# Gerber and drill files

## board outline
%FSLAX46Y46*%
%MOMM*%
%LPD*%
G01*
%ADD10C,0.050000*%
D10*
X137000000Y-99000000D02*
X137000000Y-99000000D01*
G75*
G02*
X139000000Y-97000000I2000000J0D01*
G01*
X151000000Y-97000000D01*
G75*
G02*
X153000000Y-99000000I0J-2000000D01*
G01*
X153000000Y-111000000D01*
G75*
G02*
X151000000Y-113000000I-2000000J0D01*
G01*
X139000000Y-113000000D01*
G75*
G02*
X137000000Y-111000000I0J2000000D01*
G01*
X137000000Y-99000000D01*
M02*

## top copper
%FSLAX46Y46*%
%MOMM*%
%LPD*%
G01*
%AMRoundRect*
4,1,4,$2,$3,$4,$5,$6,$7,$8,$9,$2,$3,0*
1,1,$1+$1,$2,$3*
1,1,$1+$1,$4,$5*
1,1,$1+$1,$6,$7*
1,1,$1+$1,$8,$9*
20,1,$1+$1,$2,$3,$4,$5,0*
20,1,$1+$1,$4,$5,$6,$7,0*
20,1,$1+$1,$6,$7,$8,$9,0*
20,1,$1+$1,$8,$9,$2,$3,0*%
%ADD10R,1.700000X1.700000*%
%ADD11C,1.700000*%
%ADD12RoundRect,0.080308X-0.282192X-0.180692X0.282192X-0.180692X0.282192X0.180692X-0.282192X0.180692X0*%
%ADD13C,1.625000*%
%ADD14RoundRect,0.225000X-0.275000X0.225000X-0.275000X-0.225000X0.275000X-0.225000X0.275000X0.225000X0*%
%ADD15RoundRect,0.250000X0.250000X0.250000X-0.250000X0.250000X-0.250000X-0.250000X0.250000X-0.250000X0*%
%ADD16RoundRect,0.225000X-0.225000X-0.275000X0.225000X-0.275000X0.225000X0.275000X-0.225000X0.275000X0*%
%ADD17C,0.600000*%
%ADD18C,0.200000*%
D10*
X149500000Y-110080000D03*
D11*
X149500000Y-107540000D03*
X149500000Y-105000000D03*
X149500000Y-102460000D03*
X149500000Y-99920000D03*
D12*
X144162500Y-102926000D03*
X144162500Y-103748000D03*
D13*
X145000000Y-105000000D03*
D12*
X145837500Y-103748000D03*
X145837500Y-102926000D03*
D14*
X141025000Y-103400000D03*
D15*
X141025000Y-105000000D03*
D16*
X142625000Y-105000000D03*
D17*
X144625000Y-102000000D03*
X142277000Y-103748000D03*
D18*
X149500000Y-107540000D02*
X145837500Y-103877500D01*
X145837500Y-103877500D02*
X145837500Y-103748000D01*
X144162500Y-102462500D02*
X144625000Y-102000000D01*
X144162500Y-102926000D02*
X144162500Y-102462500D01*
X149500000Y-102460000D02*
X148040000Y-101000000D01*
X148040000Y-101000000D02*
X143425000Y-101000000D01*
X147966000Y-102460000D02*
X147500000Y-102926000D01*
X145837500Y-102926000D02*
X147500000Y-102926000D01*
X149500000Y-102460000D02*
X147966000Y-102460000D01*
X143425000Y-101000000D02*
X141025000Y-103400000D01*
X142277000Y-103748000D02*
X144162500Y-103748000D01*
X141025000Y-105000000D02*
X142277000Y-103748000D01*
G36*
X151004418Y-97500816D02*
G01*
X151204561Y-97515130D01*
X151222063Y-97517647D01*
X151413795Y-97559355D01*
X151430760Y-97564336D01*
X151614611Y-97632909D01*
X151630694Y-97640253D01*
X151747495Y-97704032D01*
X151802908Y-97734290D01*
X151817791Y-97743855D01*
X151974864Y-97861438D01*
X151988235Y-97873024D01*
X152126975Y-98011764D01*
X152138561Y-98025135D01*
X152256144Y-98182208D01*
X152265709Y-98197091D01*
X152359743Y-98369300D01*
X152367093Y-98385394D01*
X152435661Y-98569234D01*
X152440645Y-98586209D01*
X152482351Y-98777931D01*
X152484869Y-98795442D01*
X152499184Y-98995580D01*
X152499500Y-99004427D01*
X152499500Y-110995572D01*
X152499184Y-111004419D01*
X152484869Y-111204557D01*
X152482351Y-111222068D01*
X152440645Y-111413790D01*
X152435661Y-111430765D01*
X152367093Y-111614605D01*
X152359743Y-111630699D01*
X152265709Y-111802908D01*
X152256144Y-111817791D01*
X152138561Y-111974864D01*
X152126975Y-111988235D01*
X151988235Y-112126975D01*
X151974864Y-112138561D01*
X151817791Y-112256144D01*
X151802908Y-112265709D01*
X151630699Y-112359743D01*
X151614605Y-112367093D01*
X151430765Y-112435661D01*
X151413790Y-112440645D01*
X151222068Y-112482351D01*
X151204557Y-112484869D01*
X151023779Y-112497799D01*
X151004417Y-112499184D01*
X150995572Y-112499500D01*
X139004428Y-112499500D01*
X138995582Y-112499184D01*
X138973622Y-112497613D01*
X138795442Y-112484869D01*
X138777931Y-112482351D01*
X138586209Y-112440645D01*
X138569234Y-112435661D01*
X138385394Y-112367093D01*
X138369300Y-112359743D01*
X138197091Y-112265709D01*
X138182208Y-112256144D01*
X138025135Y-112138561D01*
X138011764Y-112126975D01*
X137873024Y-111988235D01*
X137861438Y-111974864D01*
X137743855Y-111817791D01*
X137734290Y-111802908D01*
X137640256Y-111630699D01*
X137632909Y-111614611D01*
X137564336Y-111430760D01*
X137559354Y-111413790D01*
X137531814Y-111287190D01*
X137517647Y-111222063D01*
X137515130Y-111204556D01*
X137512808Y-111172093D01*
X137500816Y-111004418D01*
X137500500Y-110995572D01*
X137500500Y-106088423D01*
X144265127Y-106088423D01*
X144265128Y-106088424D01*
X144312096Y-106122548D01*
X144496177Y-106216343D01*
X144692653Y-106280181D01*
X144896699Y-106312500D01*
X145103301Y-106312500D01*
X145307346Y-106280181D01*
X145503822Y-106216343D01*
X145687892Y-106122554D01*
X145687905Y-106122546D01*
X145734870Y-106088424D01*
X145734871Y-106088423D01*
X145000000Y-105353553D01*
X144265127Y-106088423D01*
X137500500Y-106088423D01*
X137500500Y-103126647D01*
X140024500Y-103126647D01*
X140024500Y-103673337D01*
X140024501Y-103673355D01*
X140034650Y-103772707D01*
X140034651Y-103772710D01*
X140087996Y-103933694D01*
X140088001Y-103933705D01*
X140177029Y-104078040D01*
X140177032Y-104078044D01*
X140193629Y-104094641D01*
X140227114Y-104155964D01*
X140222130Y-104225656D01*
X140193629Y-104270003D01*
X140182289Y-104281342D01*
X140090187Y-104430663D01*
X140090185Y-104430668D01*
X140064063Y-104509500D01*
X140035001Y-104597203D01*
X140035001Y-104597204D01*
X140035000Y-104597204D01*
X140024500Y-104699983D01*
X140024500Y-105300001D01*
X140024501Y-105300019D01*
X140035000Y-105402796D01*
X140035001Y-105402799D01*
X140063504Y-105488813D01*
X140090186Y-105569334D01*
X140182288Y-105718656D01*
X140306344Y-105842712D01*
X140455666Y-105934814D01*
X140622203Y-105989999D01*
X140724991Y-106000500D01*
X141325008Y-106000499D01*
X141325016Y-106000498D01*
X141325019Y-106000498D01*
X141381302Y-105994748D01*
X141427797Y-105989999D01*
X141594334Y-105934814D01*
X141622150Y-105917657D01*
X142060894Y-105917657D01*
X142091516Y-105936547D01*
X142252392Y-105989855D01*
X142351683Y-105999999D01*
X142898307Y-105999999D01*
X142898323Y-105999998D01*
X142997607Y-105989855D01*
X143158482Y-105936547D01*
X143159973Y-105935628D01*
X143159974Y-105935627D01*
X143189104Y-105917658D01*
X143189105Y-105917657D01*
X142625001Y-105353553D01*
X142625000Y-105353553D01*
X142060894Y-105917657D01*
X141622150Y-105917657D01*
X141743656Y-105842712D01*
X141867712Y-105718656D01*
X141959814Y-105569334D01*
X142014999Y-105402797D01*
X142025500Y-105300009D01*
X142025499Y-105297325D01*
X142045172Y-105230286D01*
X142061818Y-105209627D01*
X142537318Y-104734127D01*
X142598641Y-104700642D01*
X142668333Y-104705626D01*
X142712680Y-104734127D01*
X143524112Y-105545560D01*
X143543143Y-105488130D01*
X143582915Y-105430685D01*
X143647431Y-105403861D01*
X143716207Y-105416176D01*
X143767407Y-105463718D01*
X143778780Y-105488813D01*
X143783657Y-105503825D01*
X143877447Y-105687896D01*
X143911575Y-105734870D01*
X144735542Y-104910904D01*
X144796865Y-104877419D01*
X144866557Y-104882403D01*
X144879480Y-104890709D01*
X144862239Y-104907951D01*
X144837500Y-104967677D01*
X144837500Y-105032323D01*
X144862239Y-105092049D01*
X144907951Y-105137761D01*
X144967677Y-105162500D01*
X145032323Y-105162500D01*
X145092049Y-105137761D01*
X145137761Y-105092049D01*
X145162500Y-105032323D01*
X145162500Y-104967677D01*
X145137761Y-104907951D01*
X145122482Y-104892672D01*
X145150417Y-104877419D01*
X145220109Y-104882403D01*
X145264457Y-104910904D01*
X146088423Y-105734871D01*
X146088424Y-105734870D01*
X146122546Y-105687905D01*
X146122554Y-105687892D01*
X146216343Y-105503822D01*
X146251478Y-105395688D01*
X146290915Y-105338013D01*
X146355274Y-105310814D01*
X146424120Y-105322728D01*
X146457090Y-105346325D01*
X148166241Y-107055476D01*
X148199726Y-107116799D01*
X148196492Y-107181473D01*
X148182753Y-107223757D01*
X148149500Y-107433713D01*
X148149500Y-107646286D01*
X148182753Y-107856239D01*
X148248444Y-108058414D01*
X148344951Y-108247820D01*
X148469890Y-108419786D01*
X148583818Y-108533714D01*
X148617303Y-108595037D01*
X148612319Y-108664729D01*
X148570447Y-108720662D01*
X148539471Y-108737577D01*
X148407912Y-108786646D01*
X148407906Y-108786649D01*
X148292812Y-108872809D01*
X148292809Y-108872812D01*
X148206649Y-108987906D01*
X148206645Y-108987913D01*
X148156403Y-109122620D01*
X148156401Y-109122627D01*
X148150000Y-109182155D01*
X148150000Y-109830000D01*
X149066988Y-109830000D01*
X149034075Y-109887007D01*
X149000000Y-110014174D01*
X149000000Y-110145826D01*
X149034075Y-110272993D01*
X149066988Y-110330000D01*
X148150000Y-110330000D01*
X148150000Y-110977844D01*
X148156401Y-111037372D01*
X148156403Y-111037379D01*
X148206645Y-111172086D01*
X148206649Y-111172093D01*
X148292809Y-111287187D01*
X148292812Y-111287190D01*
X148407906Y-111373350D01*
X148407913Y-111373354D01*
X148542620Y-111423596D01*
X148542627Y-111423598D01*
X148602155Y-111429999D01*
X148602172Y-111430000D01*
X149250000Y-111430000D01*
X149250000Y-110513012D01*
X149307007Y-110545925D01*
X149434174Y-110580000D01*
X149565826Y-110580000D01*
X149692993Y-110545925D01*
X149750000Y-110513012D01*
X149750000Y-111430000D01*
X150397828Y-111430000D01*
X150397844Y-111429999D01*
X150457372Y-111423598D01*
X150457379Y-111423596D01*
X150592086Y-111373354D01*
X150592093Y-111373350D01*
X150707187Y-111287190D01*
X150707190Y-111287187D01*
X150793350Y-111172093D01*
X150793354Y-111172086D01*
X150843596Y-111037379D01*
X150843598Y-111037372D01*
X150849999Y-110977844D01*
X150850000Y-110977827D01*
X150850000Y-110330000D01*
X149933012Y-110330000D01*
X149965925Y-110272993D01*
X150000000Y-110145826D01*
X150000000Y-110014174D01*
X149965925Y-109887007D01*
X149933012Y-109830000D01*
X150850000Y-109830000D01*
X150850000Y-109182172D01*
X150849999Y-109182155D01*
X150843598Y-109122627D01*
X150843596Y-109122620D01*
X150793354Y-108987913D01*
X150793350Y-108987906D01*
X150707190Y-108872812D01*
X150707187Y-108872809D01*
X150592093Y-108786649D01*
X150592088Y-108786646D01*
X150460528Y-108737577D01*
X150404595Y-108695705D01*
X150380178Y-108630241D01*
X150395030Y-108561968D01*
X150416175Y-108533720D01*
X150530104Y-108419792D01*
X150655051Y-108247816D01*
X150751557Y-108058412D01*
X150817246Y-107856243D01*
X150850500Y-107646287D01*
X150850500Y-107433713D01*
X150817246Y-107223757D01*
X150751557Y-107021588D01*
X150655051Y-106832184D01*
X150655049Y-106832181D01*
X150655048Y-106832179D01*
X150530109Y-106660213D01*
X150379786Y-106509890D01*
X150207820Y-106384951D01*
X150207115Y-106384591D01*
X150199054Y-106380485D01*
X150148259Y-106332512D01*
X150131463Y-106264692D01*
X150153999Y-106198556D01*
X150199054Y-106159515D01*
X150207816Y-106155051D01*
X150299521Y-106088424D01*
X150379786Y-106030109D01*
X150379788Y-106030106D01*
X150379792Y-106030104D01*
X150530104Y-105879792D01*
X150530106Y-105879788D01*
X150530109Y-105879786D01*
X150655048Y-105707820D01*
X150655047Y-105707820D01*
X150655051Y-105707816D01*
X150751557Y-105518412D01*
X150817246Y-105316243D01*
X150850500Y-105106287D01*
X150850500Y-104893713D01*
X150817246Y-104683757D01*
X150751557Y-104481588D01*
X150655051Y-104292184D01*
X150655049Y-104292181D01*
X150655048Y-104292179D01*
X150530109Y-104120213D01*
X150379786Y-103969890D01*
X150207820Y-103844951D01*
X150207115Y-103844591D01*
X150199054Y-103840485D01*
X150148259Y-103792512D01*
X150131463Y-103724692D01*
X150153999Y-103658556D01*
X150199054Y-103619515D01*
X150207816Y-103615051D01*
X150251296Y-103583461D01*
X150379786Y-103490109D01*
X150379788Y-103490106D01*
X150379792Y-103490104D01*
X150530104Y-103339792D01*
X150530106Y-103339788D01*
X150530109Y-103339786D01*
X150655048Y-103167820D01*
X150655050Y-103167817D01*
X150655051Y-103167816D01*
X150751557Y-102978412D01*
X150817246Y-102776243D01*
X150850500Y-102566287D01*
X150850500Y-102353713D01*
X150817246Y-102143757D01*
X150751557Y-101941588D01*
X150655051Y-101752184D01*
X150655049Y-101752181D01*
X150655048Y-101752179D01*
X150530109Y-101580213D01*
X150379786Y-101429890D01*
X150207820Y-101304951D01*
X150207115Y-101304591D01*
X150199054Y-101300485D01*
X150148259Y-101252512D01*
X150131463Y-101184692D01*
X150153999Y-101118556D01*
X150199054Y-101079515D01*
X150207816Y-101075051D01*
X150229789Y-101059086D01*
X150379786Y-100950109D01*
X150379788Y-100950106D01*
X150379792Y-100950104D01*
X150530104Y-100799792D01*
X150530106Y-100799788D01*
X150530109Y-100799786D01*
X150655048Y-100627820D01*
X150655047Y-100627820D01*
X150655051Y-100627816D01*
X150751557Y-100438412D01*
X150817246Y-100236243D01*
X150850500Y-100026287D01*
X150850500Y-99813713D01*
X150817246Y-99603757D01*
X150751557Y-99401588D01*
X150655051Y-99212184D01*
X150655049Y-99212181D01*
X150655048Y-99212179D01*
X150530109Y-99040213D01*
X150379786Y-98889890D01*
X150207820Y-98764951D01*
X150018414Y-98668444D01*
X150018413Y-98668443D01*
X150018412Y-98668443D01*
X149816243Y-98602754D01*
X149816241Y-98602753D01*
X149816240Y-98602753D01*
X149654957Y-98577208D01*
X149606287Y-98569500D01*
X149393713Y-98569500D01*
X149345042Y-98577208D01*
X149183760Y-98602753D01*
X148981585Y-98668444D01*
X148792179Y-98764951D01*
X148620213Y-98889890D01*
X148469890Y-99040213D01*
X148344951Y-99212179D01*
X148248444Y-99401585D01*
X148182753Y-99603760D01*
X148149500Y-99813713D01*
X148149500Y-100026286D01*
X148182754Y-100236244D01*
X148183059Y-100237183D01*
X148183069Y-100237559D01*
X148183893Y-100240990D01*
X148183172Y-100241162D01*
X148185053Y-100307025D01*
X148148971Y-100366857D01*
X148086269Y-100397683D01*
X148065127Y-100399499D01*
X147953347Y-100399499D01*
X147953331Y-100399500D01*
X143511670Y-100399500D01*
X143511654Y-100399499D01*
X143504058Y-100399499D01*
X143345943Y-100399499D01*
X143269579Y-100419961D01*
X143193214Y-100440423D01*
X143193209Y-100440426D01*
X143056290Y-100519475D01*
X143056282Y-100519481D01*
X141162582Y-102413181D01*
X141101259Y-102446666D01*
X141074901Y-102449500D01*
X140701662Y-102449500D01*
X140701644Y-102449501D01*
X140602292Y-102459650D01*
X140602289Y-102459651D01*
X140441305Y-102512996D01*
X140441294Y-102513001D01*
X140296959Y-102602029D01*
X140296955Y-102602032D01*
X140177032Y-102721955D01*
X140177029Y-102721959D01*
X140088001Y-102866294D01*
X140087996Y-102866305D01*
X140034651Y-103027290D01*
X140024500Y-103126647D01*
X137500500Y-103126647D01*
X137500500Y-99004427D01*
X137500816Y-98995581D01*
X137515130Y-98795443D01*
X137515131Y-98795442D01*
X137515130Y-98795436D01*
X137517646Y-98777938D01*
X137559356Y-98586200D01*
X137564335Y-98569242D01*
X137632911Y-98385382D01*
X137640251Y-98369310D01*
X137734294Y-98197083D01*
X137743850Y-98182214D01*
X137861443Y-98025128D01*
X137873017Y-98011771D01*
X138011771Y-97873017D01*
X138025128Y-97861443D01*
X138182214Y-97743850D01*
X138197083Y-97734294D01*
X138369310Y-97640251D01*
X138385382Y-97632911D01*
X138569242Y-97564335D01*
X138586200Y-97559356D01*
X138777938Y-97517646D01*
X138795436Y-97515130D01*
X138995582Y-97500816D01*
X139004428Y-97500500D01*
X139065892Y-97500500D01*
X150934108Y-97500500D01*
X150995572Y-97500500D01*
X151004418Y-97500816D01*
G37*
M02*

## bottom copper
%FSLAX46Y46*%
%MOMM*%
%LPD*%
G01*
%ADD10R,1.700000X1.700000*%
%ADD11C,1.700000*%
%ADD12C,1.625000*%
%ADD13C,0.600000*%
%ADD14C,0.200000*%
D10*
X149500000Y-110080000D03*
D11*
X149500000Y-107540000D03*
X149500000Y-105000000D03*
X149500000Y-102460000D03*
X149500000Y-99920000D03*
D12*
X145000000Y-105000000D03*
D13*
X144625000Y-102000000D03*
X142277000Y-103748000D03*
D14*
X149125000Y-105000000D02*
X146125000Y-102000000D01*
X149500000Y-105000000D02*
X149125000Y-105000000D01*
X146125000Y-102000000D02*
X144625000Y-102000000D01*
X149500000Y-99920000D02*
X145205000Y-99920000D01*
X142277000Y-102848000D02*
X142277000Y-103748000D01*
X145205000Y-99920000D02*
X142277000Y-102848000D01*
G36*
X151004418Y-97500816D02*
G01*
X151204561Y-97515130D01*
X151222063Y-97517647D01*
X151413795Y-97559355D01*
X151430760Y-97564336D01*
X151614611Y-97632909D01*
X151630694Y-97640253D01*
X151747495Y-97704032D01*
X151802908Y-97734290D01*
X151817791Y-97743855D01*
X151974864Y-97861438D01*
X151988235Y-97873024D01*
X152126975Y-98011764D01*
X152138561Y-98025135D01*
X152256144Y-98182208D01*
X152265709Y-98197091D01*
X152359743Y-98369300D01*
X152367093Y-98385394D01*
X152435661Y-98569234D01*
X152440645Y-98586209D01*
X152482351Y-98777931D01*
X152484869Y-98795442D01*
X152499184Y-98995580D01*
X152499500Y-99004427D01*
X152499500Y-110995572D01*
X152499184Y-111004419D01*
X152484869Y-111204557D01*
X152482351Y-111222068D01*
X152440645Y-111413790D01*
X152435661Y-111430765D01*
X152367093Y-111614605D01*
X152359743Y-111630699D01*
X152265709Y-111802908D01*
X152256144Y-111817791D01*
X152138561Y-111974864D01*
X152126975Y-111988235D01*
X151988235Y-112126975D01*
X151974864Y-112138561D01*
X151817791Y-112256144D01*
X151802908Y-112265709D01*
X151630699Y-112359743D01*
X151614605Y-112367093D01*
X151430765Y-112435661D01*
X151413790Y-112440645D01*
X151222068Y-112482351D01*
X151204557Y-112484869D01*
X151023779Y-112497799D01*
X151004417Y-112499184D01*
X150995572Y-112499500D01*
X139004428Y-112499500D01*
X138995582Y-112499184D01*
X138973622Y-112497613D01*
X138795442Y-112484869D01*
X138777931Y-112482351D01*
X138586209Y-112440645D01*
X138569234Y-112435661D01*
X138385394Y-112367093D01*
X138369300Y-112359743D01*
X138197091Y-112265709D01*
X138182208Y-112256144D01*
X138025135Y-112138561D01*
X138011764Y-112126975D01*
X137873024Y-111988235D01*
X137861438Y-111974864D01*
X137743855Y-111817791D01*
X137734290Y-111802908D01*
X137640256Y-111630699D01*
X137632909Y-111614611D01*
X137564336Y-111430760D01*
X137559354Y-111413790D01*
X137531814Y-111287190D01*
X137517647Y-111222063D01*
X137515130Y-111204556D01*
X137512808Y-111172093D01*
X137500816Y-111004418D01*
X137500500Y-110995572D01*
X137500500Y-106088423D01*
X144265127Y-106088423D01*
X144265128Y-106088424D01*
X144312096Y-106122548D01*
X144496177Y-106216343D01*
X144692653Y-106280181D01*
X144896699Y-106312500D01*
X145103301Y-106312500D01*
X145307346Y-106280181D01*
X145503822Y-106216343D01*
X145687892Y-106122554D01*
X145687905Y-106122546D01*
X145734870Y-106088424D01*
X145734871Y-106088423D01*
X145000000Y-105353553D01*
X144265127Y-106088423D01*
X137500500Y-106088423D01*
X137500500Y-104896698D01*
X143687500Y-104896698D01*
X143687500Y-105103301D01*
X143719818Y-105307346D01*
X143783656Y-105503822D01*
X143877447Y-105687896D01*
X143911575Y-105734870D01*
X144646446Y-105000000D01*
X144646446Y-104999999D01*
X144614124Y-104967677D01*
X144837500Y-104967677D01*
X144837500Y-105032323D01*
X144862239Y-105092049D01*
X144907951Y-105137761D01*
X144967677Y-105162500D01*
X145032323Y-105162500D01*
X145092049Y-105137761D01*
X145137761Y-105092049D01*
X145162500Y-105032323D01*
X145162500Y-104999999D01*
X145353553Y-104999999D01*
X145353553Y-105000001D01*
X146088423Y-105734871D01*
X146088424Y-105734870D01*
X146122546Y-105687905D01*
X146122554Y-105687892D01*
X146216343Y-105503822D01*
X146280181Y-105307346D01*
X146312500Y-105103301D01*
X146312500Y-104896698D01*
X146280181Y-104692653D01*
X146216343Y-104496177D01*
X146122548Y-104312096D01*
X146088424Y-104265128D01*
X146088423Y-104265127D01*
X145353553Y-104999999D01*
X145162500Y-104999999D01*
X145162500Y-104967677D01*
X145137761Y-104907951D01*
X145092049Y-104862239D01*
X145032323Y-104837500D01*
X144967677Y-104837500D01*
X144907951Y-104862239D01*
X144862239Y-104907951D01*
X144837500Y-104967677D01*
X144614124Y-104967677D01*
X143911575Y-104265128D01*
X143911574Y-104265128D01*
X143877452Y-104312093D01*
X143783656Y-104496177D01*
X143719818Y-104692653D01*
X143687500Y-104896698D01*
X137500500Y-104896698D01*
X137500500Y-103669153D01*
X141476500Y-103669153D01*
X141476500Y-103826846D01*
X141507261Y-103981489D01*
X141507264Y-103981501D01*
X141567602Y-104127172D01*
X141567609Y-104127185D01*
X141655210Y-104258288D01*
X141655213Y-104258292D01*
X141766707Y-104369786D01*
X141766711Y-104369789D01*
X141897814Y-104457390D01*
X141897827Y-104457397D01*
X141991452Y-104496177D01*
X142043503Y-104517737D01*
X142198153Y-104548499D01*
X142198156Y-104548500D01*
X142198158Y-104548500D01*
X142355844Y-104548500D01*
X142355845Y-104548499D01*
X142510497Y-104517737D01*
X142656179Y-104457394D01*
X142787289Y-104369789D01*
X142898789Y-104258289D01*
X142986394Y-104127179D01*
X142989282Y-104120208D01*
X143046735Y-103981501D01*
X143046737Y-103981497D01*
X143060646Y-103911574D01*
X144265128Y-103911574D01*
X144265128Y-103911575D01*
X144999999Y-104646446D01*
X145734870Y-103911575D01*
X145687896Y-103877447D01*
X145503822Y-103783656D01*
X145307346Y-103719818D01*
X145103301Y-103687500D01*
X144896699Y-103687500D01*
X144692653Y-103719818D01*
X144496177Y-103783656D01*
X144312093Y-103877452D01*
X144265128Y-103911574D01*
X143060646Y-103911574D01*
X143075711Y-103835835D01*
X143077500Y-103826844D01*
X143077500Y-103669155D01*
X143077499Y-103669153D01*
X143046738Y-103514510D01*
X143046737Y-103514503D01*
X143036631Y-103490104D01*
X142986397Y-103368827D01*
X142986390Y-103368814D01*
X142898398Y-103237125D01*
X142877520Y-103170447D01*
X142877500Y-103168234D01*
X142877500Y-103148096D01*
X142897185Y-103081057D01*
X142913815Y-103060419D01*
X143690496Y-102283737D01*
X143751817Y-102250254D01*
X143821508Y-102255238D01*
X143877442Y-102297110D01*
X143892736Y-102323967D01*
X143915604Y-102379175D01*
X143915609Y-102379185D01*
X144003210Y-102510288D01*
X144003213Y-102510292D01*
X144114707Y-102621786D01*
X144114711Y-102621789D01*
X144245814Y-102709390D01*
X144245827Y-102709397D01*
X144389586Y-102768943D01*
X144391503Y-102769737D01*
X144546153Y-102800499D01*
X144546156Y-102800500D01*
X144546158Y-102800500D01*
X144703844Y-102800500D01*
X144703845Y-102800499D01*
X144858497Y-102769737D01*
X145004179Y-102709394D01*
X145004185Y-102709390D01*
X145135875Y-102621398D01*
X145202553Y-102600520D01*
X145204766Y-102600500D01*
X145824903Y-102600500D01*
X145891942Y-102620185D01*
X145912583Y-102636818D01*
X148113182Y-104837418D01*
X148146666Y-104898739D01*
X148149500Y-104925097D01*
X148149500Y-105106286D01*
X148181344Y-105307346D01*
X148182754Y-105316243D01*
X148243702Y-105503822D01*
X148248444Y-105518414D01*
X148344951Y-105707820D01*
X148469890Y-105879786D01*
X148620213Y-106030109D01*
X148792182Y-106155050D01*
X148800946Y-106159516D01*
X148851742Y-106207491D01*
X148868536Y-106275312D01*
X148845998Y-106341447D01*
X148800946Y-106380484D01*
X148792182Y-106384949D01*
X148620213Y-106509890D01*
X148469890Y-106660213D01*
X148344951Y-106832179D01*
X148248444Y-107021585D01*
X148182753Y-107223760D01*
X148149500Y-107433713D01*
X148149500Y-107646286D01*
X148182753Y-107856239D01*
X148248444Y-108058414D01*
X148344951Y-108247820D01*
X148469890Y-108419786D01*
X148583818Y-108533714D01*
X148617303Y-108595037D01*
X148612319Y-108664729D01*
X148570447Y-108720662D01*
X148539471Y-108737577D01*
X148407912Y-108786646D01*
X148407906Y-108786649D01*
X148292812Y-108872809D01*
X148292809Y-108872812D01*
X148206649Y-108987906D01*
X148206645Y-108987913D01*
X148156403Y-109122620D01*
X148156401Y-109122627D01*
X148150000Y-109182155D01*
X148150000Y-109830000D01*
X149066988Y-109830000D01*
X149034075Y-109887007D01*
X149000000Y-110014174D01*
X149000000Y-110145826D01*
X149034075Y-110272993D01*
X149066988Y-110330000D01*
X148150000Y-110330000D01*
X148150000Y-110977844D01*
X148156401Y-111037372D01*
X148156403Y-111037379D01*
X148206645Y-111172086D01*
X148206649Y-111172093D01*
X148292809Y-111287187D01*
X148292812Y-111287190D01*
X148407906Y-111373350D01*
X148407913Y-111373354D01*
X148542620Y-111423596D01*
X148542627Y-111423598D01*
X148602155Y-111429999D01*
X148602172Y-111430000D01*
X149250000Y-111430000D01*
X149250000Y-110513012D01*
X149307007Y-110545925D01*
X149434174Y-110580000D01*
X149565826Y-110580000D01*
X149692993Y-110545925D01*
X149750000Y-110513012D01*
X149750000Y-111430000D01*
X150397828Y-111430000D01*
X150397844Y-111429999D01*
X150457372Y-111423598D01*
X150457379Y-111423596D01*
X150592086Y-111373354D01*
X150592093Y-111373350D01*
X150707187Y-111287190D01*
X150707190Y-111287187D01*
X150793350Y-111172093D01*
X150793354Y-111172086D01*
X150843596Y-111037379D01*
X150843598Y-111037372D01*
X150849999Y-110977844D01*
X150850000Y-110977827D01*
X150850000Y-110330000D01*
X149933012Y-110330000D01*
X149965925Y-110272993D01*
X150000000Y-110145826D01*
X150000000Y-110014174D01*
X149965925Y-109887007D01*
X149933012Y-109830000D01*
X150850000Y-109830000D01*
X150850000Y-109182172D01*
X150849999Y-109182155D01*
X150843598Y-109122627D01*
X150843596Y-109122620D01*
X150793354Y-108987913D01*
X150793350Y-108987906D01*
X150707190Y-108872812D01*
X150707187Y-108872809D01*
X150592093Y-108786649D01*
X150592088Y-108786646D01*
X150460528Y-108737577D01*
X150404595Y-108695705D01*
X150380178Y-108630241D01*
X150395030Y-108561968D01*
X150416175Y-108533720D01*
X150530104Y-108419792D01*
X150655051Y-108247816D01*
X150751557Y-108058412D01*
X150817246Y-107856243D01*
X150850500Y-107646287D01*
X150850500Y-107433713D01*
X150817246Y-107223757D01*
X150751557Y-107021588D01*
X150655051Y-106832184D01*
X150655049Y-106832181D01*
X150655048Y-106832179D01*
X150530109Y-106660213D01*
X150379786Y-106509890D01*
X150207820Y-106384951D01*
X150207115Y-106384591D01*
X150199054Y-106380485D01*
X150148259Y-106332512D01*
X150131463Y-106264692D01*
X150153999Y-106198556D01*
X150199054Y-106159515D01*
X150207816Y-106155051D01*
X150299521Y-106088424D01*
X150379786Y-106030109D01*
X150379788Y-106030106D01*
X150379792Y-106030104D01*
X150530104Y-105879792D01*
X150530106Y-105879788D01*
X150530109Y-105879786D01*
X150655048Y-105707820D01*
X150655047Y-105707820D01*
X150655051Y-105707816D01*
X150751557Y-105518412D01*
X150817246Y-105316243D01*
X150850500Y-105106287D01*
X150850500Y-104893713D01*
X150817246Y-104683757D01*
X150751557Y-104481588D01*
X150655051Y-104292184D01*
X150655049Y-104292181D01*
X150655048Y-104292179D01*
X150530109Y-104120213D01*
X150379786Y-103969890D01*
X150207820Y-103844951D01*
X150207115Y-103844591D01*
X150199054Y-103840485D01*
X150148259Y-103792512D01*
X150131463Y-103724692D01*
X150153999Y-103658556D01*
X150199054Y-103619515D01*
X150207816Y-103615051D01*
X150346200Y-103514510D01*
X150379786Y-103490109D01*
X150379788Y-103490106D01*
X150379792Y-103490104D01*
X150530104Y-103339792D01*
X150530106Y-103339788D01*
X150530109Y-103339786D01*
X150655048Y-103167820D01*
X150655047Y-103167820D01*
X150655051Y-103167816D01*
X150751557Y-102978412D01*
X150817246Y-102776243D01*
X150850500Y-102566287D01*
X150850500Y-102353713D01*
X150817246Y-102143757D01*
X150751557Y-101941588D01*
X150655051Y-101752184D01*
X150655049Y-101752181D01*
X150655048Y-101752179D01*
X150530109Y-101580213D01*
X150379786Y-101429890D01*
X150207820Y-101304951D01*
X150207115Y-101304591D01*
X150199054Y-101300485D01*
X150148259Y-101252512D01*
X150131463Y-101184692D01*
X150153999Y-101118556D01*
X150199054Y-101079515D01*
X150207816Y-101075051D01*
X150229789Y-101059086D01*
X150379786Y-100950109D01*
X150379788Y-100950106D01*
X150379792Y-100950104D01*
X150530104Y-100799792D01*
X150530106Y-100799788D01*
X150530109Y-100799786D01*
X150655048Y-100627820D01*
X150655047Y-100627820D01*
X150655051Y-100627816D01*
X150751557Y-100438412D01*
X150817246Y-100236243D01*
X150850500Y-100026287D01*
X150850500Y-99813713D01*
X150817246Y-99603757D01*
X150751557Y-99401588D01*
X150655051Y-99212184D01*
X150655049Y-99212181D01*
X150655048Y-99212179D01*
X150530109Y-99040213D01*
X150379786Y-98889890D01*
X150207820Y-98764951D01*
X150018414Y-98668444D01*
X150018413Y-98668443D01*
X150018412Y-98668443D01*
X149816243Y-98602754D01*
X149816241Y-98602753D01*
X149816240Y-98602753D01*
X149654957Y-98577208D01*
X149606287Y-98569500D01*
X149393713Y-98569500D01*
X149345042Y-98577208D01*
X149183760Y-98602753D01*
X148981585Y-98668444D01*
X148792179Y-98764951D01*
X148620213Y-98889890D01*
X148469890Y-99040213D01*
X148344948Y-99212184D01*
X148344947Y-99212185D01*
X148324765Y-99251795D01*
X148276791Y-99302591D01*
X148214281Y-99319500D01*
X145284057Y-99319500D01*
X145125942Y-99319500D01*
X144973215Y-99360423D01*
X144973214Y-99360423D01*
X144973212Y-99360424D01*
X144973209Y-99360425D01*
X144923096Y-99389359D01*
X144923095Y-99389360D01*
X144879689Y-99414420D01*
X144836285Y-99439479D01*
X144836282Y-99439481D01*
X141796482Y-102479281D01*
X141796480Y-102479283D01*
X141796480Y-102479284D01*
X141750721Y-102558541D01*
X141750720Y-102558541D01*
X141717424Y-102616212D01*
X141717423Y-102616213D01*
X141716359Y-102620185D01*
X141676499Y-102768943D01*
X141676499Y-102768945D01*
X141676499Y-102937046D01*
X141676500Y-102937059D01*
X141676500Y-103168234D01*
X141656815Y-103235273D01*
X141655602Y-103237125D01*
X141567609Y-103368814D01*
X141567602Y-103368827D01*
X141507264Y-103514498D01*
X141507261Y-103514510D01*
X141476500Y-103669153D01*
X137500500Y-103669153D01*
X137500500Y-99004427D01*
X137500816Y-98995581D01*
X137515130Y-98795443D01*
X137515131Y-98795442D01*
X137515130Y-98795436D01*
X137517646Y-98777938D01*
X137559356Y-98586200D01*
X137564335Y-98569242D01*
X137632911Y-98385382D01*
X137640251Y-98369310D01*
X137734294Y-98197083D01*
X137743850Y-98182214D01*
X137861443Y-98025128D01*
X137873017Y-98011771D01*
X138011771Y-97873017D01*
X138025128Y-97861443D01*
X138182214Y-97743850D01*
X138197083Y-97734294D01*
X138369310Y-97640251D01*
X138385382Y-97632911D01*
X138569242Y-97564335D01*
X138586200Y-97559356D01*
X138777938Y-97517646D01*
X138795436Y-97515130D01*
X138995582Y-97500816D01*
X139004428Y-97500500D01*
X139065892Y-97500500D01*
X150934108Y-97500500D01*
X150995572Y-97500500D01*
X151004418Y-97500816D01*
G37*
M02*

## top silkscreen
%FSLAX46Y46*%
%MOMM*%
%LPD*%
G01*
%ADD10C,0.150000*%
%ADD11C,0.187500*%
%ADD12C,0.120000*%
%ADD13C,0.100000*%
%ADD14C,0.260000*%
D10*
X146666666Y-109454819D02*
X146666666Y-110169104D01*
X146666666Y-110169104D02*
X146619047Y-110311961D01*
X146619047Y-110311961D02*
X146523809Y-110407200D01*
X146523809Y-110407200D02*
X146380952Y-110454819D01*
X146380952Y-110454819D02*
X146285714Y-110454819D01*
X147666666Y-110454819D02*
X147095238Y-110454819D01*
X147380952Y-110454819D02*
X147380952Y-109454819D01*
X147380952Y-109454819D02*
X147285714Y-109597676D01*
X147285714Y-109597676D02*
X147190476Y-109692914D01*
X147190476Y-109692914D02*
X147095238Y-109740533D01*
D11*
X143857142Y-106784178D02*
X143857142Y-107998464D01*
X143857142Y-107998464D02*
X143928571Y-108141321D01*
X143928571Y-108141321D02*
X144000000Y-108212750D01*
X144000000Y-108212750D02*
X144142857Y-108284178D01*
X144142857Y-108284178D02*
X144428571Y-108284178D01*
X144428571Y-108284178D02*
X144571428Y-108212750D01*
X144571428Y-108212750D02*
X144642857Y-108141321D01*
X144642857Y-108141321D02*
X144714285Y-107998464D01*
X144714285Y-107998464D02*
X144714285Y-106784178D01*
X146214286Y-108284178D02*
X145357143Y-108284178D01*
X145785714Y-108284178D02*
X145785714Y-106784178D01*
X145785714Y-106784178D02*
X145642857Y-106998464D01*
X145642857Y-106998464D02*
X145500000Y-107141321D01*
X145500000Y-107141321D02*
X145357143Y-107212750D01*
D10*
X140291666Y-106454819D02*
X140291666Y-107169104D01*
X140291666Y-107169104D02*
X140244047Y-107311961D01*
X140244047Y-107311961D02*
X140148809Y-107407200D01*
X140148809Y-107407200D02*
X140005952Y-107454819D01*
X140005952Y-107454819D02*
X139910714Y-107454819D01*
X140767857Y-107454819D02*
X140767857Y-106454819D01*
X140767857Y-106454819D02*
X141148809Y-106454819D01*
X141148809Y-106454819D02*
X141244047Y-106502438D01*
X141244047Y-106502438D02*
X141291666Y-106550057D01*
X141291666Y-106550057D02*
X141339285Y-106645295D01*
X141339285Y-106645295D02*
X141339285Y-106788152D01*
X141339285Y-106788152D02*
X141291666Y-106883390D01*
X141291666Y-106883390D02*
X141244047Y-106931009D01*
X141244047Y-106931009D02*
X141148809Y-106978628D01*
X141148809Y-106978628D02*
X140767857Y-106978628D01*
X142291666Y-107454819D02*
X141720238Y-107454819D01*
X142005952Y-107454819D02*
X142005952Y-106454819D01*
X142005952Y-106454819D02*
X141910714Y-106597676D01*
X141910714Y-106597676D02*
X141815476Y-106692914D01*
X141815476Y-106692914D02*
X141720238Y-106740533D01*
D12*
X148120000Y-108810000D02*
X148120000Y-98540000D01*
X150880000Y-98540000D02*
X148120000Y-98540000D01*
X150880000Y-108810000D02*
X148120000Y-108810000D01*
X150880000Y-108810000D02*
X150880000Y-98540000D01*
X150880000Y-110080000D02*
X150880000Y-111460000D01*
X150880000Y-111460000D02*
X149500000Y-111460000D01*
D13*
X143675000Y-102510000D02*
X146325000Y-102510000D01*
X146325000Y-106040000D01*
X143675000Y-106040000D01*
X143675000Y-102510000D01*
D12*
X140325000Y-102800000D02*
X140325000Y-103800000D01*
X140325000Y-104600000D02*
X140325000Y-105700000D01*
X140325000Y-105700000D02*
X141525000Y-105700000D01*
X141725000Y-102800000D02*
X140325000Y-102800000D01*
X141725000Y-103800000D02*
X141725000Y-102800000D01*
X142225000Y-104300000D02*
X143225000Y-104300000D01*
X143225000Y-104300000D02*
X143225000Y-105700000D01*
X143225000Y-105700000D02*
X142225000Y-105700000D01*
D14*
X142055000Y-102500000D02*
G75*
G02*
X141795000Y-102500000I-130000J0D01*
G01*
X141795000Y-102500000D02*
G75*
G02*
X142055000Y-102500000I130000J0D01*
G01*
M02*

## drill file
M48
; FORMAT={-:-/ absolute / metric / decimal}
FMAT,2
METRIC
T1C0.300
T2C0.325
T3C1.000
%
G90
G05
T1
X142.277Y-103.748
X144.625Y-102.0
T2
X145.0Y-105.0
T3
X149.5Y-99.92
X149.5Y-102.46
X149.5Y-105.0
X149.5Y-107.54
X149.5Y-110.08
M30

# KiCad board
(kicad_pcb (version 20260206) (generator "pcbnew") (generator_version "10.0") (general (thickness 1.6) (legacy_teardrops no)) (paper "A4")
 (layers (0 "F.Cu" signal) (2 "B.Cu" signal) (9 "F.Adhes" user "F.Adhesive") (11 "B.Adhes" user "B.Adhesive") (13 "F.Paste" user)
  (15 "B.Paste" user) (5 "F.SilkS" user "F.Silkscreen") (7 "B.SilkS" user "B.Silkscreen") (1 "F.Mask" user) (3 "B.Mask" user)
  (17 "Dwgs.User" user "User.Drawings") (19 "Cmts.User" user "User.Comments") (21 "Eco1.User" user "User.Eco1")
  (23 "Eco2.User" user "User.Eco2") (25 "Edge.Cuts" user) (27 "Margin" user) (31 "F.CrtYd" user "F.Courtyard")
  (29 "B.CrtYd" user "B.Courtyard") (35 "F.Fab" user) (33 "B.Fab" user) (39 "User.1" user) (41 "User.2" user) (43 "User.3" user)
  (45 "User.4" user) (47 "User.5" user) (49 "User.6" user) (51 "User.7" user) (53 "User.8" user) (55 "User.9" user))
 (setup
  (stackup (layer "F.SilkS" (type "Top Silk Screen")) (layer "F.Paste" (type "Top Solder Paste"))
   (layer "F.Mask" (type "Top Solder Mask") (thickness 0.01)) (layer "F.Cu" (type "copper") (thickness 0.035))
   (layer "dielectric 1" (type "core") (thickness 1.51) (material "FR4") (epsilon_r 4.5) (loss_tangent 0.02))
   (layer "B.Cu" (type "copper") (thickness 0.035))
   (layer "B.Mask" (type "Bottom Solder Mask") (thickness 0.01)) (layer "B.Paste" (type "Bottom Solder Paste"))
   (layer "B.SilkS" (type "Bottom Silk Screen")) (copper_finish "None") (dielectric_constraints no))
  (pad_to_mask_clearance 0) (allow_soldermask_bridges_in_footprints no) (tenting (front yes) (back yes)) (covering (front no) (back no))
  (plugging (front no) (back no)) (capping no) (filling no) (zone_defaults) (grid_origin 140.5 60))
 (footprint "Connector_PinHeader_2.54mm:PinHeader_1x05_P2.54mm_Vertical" (layer "F.Cu") (at 149.5 110.08 180)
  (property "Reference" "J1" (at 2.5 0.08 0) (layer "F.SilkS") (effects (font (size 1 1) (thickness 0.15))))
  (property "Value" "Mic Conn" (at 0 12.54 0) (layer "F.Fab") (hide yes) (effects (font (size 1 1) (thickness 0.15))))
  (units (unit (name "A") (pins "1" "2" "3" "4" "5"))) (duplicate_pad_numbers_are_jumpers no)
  (fp_line (start 1.38 1.27) (end 1.38 11.54) (stroke (width 0.12) (type solid)) (layer "F.SilkS"))
  (fp_line (start -1.38 11.54) (end 1.38 11.54) (stroke (width 0.12) (type solid)) (layer "F.SilkS"))
  (fp_line (start -1.38 1.27) (end 1.38 1.27) (stroke (width 0.12) (type solid)) (layer "F.SilkS"))
  (fp_line (start -1.38 1.27) (end -1.38 11.54) (stroke (width 0.12) (type solid)) (layer "F.SilkS"))
  (fp_line (start -1.38 0) (end -1.38 -1.38) (stroke (width 0.12) (type solid)) (layer "F.SilkS"))
  (fp_line (start -1.38 -1.38) (end 0 -1.38) (stroke (width 0.12) (type solid)) (layer "F.SilkS"))
  (pad "1" thru_hole rect (at 0 0 180) (size 1.7 1.7) (drill 1) (layers "*.Cu" "*.Mask") (remove_unused_layers no) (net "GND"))
  (pad "2" thru_hole circle (at 0 2.54 180) (size 1.7 1.7) (drill 1) (layers "*.Cu" "*.Mask") (remove_unused_layers no) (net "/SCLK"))
  (pad "3" thru_hole circle (at 0 5.08 180) (size 1.7 1.7) (drill 1) (layers "*.Cu" "*.Mask") (remove_unused_layers no) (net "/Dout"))
  (pad "4" thru_hole circle (at 0 7.62 180) (size 1.7 1.7) (drill 1) (layers "*.Cu" "*.Mask") (remove_unused_layers no) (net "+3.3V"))
  (pad "5" thru_hole circle (at 0 10.16 180) (size 1.7 1.7) (drill 1) (layers "*.Cu" "*.Mask") (remove_unused_layers no) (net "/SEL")))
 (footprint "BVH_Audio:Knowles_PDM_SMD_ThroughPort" (layer "F.Cu") (at 145 105)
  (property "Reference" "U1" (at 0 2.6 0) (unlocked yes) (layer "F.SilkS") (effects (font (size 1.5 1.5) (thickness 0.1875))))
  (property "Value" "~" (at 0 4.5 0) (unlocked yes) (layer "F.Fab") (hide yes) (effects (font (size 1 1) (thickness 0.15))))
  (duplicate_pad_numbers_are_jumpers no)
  (fp_rect (start -1.325 -2.49) (end 1.325 1.04) (stroke (width 0.1) (type solid)) (fill no) (layer "F.SilkS"))
  (pad "1" smd roundrect (at -0.8375 -2.074) (size 0.725 0.522) (layers "F.Cu" "F.Mask" "F.Paste") (roundrect_rratio 0.1538461538)
   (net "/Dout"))
  (pad "2" smd roundrect (at -0.8375 -1.252) (size 0.725 0.522) (layers "F.Cu" "F.Mask" "F.Paste") (roundrect_rratio 0.1538461538)
   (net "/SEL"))
  (pad "3" thru_hole circle (at 0 0) (size 1.625 1.625) (drill 0.325) (layers "*.Cu") (remove_unused_layers no) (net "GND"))
  (pad "4" smd roundrect (at 0.8375 -1.252) (size 0.725 0.522) (layers "F.Cu" "F.Mask" "F.Paste") (roundrect_rratio 0.1538461538)
   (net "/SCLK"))
  (pad "5" smd roundrect (at 0.8375 -2.074) (size 0.725 0.522) (layers "F.Cu" "F.Mask" "F.Paste") (roundrect_rratio 0.1538461538)
   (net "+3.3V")))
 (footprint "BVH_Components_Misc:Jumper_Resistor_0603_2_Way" (layer "F.Cu") (at 141.025 105)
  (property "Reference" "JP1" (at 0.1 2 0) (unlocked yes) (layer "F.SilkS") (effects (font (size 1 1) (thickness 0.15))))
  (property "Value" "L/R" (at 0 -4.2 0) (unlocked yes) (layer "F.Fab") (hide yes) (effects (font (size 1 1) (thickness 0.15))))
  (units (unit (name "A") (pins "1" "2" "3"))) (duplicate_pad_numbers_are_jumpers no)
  (fp_line (start -0.7 -2.2) (end -0.7 -1.2) (stroke (width 0.12) (type default)) (layer "F.SilkS"))
  (fp_line (start -0.7 -0.4) (end -0.7 0.7) (stroke (width 0.12) (type default)) (layer "F.SilkS"))
  (fp_line (start -0.7 0.7) (end 0.5 0.7) (stroke (width 0.12) (type default)) (layer "F.SilkS"))
  (fp_line (start 0.7 -2.2) (end -0.7 -2.2) (stroke (width 0.12) (type default)) (layer "F.SilkS"))
  (fp_line (start 0.7 -1.2) (end 0.7 -2.2) (stroke (width 0.12) (type default)) (layer "F.SilkS"))
  (fp_line (start 1.2 -0.7) (end 2.2 -0.7) (stroke (width 0.12) (type default)) (layer "F.SilkS"))
  (fp_line (start 2.2 -0.7) (end 2.2 0.7) (stroke (width 0.12) (type default)) (layer "F.SilkS"))
  (fp_line (start 2.2 0.7) (end 1.2 0.7) (stroke (width 0.12) (type default)) (layer "F.SilkS"))
  (fp_circle (center 0.9 -2.5) (end 1.1 -2.5) (stroke (width 0.12) (type solid)) (fill yes) (layer "F.SilkS"))
  (pad "1" smd roundrect (at 0 -1.6 270) (size 0.9 1) (layers "F.Cu" "F.Mask") (roundrect_rratio 0.25) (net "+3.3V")
   (thermal_bridge_angle 45))
  (pad "2" smd roundrect (at 0 0 180) (size 1 1) (layers "F.Cu" "F.Mask") (roundrect_rratio 0.25) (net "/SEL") (thermal_bridge_angle 45))
  (pad "3" smd roundrect (at 1.6 0) (size 0.9 1) (layers "F.Cu" "F.Mask") (roundrect_rratio 0.25) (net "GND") (thermal_bridge_angle 45)))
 (gr_rect (start 137 97) (end 153 113) (radius 2) (stroke (width 0.05) (type solid)) (fill no) (layer "Edge.Cuts"))
 (segment (start 149.5 107.54) (end 145.8375 103.8775) (width 0.2) (layer "F.Cu") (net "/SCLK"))
 (segment (start 145.8375 103.8775) (end 145.8375 103.748) (width 0.2) (layer "F.Cu") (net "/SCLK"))
 (segment (start 144.1625 102.4625) (end 144.625 102) (width 0.2) (layer "F.Cu") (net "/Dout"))
 (segment (start 144.1625 102.926) (end 144.1625 102.4625) (width 0.2) (layer "F.Cu") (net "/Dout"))
 (via (at 144.625 102) (size 0.6) (drill 0.3) (layers "F.Cu" "B.Cu") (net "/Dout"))
 (segment (start 149.125 105) (end 146.125 102) (width 0.2) (layer "B.Cu") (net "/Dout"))
 (segment (start 149.5 105) (end 149.125 105) (width 0.2) (layer "B.Cu") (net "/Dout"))
 (segment (start 146.125 102) (end 144.625 102) (width 0.2) (layer "B.Cu") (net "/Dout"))
 (segment (start 149.5 102.46) (end 148.04 101) (width 0.2) (layer "F.Cu") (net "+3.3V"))
 (segment (start 148.04 101) (end 143.425 101) (width 0.2) (layer "F.Cu") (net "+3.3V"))
 (segment (start 147.966 102.46) (end 147.5 102.926) (width 0.2) (layer "F.Cu") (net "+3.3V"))
 (segment (start 145.8375 102.926) (end 147.5 102.926) (width 0.2) (layer "F.Cu") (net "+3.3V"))
 (segment (start 149.5 102.46) (end 147.966 102.46) (width 0.2) (layer "F.Cu") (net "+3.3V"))
 (segment (start 143.425 101) (end 141.025 103.4) (width 0.2) (layer "F.Cu") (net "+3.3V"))
 (segment (start 142.277 103.748) (end 144.1625 103.748) (width 0.2) (layer "F.Cu") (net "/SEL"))
 (segment (start 141.025 105) (end 142.277 103.748) (width 0.2) (layer "F.Cu") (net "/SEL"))
 (via (at 142.277 103.748) (size 0.6) (drill 0.3) (layers "F.Cu" "B.Cu") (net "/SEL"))
 (segment (start 149.5 99.92) (end 145.205 99.92) (width 0.2) (layer "B.Cu") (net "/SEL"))
 (segment (start 142.277 102.848) (end 142.277 103.748) (width 0.2) (layer "B.Cu") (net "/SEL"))
 (segment (start 145.205 99.92) (end 142.277 102.848) (width 0.2) (layer "B.Cu") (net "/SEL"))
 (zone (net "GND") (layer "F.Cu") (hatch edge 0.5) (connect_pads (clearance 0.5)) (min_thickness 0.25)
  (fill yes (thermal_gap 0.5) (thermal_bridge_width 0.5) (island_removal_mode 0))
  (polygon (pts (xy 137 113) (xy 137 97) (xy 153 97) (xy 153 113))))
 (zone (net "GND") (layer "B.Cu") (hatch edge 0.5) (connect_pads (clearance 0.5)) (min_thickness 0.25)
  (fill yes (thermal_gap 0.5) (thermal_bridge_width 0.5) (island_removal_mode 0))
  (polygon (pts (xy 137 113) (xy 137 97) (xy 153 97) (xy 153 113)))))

